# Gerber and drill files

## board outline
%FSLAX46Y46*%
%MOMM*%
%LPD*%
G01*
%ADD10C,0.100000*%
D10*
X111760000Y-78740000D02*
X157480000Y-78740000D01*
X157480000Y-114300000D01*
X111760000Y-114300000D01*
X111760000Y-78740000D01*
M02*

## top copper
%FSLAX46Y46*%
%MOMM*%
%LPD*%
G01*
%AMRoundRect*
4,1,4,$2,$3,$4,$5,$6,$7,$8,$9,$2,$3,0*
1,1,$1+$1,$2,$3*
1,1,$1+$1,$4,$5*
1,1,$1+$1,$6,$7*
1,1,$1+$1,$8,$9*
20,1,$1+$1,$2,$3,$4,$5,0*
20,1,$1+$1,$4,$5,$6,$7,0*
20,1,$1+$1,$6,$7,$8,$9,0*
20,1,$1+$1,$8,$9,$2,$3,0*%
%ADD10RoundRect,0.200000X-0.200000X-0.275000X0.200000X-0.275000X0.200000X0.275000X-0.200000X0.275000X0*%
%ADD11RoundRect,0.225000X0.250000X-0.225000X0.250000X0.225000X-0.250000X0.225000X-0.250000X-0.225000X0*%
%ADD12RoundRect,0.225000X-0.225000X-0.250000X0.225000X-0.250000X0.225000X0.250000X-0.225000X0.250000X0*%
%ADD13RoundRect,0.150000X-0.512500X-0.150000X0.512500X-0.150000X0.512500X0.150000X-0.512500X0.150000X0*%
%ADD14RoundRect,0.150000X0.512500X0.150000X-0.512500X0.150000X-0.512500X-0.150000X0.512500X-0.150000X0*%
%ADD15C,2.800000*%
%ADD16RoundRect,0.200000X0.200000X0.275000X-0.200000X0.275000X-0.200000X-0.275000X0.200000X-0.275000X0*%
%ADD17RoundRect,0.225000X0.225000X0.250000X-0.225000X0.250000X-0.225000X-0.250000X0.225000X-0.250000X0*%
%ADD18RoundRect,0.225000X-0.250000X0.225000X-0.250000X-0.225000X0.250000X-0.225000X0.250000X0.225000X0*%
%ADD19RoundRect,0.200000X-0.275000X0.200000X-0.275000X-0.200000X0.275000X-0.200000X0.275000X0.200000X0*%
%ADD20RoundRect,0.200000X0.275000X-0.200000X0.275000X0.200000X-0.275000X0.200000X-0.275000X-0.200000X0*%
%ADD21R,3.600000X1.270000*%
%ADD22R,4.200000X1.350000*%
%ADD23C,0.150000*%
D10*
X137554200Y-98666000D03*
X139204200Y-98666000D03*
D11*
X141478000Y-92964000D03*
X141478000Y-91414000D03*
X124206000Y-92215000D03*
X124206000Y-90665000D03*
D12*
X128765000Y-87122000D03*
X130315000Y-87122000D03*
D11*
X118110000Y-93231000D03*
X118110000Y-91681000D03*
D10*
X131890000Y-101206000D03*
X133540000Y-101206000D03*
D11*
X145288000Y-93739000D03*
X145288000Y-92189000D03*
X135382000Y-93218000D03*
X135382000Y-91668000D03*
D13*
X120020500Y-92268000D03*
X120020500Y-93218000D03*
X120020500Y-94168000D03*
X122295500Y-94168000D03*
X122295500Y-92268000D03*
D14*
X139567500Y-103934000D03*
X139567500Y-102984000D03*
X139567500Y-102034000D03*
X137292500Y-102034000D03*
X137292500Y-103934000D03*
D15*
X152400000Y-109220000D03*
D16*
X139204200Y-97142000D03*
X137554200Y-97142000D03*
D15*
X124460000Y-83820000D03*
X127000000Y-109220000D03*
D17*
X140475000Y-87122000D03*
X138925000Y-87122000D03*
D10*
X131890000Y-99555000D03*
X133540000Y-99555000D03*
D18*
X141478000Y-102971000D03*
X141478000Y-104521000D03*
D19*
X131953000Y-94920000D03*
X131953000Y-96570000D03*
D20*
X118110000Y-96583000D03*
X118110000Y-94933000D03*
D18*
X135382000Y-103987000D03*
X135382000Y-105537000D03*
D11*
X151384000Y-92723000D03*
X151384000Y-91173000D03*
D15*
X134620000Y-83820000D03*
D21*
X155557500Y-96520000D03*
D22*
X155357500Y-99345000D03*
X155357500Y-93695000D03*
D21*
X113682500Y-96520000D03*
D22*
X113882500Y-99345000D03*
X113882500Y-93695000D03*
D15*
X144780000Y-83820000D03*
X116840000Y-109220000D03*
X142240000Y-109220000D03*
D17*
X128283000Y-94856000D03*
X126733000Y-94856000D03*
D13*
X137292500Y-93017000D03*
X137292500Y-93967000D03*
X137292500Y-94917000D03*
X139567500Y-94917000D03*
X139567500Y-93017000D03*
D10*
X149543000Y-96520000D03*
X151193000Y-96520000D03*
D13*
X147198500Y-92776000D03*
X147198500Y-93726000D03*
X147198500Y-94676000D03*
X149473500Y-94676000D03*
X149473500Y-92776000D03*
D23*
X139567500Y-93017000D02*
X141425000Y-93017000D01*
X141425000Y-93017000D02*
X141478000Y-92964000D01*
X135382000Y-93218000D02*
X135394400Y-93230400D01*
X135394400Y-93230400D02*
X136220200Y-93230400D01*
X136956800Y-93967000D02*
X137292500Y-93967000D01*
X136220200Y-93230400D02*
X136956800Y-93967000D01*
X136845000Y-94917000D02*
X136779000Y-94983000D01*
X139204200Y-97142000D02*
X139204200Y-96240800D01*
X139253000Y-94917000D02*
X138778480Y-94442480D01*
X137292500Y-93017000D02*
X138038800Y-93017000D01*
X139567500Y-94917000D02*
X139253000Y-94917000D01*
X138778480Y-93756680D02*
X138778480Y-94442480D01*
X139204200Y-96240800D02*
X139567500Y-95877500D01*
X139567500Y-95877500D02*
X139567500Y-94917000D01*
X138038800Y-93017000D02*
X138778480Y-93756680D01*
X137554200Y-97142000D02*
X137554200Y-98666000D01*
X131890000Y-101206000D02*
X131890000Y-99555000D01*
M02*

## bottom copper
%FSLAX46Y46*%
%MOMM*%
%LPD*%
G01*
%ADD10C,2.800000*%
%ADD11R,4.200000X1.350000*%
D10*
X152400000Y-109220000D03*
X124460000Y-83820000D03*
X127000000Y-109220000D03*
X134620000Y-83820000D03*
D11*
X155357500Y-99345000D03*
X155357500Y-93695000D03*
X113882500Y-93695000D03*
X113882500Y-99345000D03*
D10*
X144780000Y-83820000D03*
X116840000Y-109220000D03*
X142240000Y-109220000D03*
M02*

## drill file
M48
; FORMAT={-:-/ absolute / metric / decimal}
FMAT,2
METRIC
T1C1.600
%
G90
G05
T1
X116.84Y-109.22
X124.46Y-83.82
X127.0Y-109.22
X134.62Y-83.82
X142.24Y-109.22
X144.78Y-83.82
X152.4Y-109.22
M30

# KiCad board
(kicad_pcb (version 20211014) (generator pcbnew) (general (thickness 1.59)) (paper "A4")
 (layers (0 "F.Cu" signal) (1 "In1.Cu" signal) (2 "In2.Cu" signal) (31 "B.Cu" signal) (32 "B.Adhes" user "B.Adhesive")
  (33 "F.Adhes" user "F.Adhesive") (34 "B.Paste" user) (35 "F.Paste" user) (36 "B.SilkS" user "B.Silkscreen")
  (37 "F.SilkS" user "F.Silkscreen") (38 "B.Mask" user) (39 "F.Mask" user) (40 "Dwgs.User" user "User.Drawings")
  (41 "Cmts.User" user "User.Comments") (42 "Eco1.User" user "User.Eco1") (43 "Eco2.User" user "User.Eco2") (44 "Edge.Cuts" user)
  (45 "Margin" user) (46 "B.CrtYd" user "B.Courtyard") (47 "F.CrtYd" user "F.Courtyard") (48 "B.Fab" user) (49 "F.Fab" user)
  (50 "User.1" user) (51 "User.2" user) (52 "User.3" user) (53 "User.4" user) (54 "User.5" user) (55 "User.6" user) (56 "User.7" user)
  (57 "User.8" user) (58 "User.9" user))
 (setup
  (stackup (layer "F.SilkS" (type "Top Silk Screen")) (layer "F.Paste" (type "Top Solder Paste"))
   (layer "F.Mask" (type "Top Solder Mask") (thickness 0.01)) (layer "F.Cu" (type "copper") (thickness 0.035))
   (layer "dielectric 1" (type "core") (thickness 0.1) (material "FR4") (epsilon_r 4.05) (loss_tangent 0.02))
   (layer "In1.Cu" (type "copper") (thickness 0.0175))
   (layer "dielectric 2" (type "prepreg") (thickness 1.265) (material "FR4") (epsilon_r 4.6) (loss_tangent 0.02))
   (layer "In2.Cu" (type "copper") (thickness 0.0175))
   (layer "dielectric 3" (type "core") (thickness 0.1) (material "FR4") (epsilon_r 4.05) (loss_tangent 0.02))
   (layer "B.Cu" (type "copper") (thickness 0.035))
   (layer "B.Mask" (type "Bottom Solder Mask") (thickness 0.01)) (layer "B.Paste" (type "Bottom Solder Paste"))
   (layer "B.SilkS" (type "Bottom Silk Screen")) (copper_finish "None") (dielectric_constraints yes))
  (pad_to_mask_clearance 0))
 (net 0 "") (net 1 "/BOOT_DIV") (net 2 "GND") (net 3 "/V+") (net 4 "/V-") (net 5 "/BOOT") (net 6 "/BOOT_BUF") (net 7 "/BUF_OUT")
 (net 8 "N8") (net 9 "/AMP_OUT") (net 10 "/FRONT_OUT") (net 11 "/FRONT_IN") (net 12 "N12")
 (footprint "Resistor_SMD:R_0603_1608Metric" (layer "F.Cu") (at 138.3792 98.666)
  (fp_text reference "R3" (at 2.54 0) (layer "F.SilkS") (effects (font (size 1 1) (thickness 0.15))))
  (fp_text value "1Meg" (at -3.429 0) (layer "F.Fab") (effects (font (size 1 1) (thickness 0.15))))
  (pad "1" smd roundrect (at -0.825 0) (size 0.8 0.95) (layers "F.Cu" "F.Paste" "F.Mask") (roundrect_rratio 0.25) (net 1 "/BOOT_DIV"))
  (pad "2" smd roundrect (at 0.825 0) (size 0.8 0.95) (layers "F.Cu" "F.Paste" "F.Mask") (roundrect_rratio 0.25) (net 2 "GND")))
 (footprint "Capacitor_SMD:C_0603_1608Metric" (layer "F.Cu") (at 141.478 92.189 90)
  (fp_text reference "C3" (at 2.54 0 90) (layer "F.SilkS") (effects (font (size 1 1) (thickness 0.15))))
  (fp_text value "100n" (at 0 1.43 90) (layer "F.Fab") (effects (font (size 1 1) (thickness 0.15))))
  (pad "1" smd roundrect (at -0.775 0 90) (size 0.9 0.95) (layers "F.Cu" "F.Paste" "F.Mask") (roundrect_rratio 0.25) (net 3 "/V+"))
  (pad "2" smd roundrect (at 0.775 0 90) (size 0.9 0.95) (layers "F.Cu" "F.Paste" "F.Mask") (roundrect_rratio 0.25) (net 2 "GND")))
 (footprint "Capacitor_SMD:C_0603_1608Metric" (layer "F.Cu") (at 124.206 91.44 90)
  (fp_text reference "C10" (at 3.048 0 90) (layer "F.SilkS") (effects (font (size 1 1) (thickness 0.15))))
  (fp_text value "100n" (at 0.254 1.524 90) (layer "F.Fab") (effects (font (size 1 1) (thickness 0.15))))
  (pad "1" smd roundrect (at -0.775 0 90) (size 0.9 0.95) (layers "F.Cu" "F.Paste" "F.Mask") (roundrect_rratio 0.25) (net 3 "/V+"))
  (pad "2" smd roundrect (at 0.775 0 90) (size 0.9 0.95) (layers "F.Cu" "F.Paste" "F.Mask") (roundrect_rratio 0.25) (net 2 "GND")))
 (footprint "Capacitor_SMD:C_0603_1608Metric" (layer "F.Cu") (at 129.54 87.122)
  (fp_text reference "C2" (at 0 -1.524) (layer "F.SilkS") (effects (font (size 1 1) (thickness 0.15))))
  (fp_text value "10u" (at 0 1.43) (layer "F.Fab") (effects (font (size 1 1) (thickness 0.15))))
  (pad "1" smd roundrect (at -0.775 0) (size 0.9 0.95) (layers "F.Cu" "F.Paste" "F.Mask") (roundrect_rratio 0.25) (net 3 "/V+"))
  (pad "2" smd roundrect (at 0.775 0) (size 0.9 0.95) (layers "F.Cu" "F.Paste" "F.Mask") (roundrect_rratio 0.25) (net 2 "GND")))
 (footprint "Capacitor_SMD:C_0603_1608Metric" (layer "F.Cu") (at 118.11 92.456 90)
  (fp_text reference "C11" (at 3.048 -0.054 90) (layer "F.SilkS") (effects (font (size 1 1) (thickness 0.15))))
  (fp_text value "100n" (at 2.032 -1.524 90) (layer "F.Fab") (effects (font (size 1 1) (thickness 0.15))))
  (pad "1" smd roundrect (at -0.775 0 90) (size 0.9 0.95) (layers "F.Cu" "F.Paste" "F.Mask") (roundrect_rratio 0.25) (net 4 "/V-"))
  (pad "2" smd roundrect (at 0.775 0 90) (size 0.9 0.95) (layers "F.Cu" "F.Paste" "F.Mask") (roundrect_rratio 0.25) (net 2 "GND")))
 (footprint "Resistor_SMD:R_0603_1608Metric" (layer "F.Cu") (at 132.715 101.206)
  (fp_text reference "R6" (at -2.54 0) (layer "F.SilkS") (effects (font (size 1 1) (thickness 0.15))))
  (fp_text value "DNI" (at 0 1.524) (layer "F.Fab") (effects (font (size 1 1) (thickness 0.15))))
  (pad "1" smd roundrect (at -0.825 0) (size 0.8 0.95) (layers "F.Cu" "F.Paste" "F.Mask") (roundrect_rratio 0.25) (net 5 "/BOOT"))
  (pad "2" smd roundrect (at 0.825 0) (size 0.8 0.95) (layers "F.Cu" "F.Paste" "F.Mask") (roundrect_rratio 0.25) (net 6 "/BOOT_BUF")))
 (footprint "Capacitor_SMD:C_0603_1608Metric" (layer "F.Cu") (at 145.288 92.964 90)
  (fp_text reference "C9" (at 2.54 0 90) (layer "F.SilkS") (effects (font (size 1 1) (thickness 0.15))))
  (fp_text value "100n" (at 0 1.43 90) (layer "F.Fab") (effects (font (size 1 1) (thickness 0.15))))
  (pad "1" smd roundrect (at -0.775 0 90) (size 0.9 0.95) (layers "F.Cu" "F.Paste" "F.Mask") (roundrect_rratio 0.25) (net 4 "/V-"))
  (pad "2" smd roundrect (at 0.775 0 90) (size 0.9 0.95) (layers "F.Cu" "F.Paste" "F.Mask") (roundrect_rratio 0.25) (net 2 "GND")))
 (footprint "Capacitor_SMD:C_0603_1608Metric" (layer "F.Cu") (at 135.382 92.443 90)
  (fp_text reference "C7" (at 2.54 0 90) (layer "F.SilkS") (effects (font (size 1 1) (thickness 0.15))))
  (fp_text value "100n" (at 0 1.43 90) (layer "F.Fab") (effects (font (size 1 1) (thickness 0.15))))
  (pad "1" smd roundrect (at -0.775 0 90) (size 0.9 0.95) (layers "F.Cu" "F.Paste" "F.Mask") (roundrect_rratio 0.25) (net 4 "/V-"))
  (pad "2" smd roundrect (at 0.775 0 90) (size 0.9 0.95) (layers "F.Cu" "F.Paste" "F.Mask") (roundrect_rratio 0.25) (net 2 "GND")))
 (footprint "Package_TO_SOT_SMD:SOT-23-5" (layer "F.Cu") (at 121.158 93.218)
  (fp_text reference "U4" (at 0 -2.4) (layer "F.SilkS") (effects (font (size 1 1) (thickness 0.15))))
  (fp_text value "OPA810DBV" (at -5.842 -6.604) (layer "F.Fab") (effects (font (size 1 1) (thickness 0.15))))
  (pad "1" smd roundrect (at -1.1375 -0.95) (size 1.325 0.6) (layers "F.Cu" "F.Paste" "F.Mask") (roundrect_rratio 0.25) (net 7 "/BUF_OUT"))
  (pad "2" smd roundrect (at -1.1375 0) (size 1.325 0.6) (layers "F.Cu" "F.Paste" "F.Mask") (roundrect_rratio 0.25) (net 4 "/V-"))
  (pad "3" smd roundrect (at -1.1375 0.95) (size 1.325 0.6) (layers "F.Cu" "F.Paste" "F.Mask") (roundrect_rratio 0.25) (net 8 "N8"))
  (pad "4" smd roundrect (at 1.1375 0.95) (size 1.325 0.6) (layers "F.Cu" "F.Paste" "F.Mask") (roundrect_rratio 0.25) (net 7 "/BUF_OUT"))
  (pad "5" smd roundrect (at 1.1375 -0.95) (size 1.325 0.6) (layers "F.Cu" "F.Paste" "F.Mask") (roundrect_rratio 0.25) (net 3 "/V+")))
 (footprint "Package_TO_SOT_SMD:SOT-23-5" (layer "F.Cu") (at 138.43 102.984 180)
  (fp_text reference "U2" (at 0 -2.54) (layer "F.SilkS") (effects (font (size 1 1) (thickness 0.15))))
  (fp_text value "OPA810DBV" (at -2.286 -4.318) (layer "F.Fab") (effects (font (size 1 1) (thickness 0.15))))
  (pad "1" smd roundrect (at -1.1375 -0.95 180) (size 1.325 0.6) (layers "F.Cu" "F.Paste" "F.Mask") (roundrect_rratio 0.25)
   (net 6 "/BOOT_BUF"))
  (pad "2" smd roundrect (at -1.1375 0 180) (size 1.325 0.6) (layers "F.Cu" "F.Paste" "F.Mask") (roundrect_rratio 0.25) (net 4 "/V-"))
  (pad "3" smd roundrect (at -1.1375 0.95 180) (size 1.325 0.6) (layers "F.Cu" "F.Paste" "F.Mask") (roundrect_rratio 0.25)
   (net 1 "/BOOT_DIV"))
  (pad "4" smd roundrect (at 1.1375 0.95 180) (size 1.325 0.6) (layers "F.Cu" "F.Paste" "F.Mask") (roundrect_rratio 0.25)
   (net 6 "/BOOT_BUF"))
  (pad "5" smd roundrect (at 1.1375 -0.95 180) (size 1.325 0.6) (layers "F.Cu" "F.Paste" "F.Mask") (roundrect_rratio 0.25) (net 3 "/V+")))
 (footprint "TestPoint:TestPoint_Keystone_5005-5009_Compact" (layer "F.Cu") (at 152.4 109.22)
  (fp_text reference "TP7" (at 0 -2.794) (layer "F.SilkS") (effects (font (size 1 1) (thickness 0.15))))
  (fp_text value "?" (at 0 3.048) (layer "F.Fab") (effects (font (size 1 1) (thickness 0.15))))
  (pad "1" thru_hole circle (at 0 0) (size 2.8 2.8) (drill 1.6) (layers *.Cu *.Mask) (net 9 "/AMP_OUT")))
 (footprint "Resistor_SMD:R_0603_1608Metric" (layer "F.Cu") (at 138.3792 97.142 180)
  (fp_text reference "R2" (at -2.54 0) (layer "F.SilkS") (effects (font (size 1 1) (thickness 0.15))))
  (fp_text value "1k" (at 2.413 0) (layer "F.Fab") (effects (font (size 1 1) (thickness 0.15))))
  (pad "1" smd roundrect (at -0.825 0 180) (size 0.8 0.95) (layers "F.Cu" "F.Paste" "F.Mask") (roundrect_rratio 0.25) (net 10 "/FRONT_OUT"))
  (pad "2" smd roundrect (at 0.825 0 180) (size 0.8 0.95) (layers "F.Cu" "F.Paste" "F.Mask") (roundrect_rratio 0.25) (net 1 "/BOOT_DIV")))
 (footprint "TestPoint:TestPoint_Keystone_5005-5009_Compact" (layer "F.Cu") (at 124.46 83.82)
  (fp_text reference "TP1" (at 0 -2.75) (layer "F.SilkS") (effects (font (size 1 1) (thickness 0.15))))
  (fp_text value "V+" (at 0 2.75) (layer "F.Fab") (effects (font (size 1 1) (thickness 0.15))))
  (pad "1" thru_hole circle (at 0 0) (size 2.8 2.8) (drill 1.6) (layers *.Cu *.Mask) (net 3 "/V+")))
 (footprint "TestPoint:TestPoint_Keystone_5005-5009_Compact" (layer "F.Cu") (at 127 109.22)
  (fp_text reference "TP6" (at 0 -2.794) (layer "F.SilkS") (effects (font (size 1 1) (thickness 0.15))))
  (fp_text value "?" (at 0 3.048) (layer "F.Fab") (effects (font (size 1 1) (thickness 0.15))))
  (pad "1" thru_hole circle (at 0 0) (size 2.8 2.8) (drill 1.6) (layers *.Cu *.Mask) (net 6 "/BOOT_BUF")))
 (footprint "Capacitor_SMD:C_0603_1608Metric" (layer "F.Cu") (at 139.7 87.122 180)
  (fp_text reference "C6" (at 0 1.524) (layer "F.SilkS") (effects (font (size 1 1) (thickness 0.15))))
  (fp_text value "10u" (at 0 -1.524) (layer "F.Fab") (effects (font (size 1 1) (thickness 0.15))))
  (pad "1" smd roundrect (at -0.775 0 180) (size 0.9 0.95) (layers "F.Cu" "F.Paste" "F.Mask") (roundrect_rratio 0.25) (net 4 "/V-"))
  (pad "2" smd roundrect (at 0.775 0 180) (size 0.9 0.95) (layers "F.Cu" "F.Paste" "F.Mask") (roundrect_rratio 0.25) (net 2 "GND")))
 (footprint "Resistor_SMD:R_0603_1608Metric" (layer "F.Cu") (at 132.715 99.555)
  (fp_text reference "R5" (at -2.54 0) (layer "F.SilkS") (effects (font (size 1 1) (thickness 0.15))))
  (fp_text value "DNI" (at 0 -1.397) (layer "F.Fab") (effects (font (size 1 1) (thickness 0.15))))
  (pad "1" smd roundrect (at -0.825 0) (size 0.8 0.95) (layers "F.Cu" "F.Paste" "F.Mask") (roundrect_rratio 0.25) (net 5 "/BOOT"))
  (pad "2" smd roundrect (at 0.825 0) (size 0.8 0.95) (layers "F.Cu" "F.Paste" "F.Mask") (roundrect_rratio 0.25) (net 1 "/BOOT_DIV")))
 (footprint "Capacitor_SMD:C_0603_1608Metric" (layer "F.Cu") (at 141.478 103.746 -90)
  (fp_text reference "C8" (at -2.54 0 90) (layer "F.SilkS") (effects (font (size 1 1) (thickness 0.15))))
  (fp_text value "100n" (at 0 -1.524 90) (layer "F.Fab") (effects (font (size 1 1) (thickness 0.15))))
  (pad "1" smd roundrect (at -0.775 0 270) (size 0.9 0.95) (layers "F.Cu" "F.Paste" "F.Mask") (roundrect_rratio 0.25) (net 4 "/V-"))
  (pad "2" smd roundrect (at 0.775 0 270) (size 0.9 0.95) (layers "F.Cu" "F.Paste" "F.Mask") (roundrect_rratio 0.25) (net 2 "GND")))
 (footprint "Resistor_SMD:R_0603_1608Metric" (layer "F.Cu") (at 131.953 95.745 -90)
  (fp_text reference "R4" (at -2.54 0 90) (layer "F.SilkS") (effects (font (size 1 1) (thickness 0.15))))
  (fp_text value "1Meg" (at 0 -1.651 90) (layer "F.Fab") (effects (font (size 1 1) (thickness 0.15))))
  (pad "1" smd roundrect (at -0.825 0 270) (size 0.8 0.95) (layers "F.Cu" "F.Paste" "F.Mask") (roundrect_rratio 0.25) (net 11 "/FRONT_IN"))
  (pad "2" smd roundrect (at 0.825 0 270) (size 0.8 0.95) (layers "F.Cu" "F.Paste" "F.Mask") (roundrect_rratio 0.25) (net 5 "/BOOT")))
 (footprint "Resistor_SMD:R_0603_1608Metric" (layer "F.Cu") (at 118.11 95.758 90)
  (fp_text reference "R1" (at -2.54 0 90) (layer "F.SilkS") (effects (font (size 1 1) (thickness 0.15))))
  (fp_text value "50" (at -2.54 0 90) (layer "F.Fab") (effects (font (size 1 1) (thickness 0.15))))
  (pad "1" smd roundrect (at -0.825 0 90) (size 0.8 0.95) (layers "F.Cu" "F.Paste" "F.Mask") (roundrect_rratio 0.25) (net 8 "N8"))
  (pad "2" smd roundrect (at 0.825 0 90) (size 0.8 0.95) (layers "F.Cu" "F.Paste" "F.Mask") (roundrect_rratio 0.25) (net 2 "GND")))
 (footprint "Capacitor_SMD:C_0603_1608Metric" (layer "F.Cu") (at 135.382 104.762 -90)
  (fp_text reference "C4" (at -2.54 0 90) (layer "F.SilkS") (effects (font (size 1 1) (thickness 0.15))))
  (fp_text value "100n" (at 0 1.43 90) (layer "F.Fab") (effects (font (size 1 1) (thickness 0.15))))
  (pad "1" smd roundrect (at -0.775 0 270) (size 0.9 0.95) (layers "F.Cu" "F.Paste" "F.Mask") (roundrect_rratio 0.25) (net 3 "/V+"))
  (pad "2" smd roundrect (at 0.775 0 270) (size 0.9 0.95) (layers "F.Cu" "F.Paste" "F.Mask") (roundrect_rratio 0.25) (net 2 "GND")))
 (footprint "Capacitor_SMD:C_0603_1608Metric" (layer "F.Cu") (at 151.384 91.948 90)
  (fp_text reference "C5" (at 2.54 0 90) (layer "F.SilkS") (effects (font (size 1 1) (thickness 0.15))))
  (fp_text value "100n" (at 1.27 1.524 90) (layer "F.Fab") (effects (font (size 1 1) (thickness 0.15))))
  (pad "1" smd roundrect (at -0.775 0 90) (size 0.9 0.95) (layers "F.Cu" "F.Paste" "F.Mask") (roundrect_rratio 0.25) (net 3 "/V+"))
  (pad "2" smd roundrect (at 0.775 0 90) (size 0.9 0.95) (layers "F.Cu" "F.Paste" "F.Mask") (roundrect_rratio 0.25) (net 2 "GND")))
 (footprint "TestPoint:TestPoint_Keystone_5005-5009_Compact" (layer "F.Cu") (at 134.62 83.82)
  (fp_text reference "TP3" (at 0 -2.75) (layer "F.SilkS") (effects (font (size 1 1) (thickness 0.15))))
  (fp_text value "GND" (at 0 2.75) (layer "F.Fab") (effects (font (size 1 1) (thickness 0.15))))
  (pad "1" thru_hole circle (at 0 0) (size 2.8 2.8) (drill 1.6) (layers *.Cu *.Mask) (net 2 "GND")))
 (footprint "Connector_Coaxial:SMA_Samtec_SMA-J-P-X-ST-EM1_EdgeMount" (layer "F.Cu") (at 155.3575 96.52 90)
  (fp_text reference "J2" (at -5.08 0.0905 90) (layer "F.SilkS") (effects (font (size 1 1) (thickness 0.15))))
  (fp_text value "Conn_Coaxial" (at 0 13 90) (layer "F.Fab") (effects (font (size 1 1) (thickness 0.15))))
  (pad "1" smd rect (at 0 0.2 90) (size 1.27 3.6) (layers "F.Cu" "F.Paste" "F.Mask") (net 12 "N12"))
  (pad "2" smd rect (at -2.825 0 90) (size 1.35 4.2) (layers "F.Cu" "F.Paste" "F.Mask") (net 2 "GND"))
  (pad "2" smd rect (at 2.825 0 90) (size 1.35 4.2) (layers "F.Cu" "F.Paste" "F.Mask") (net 2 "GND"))
  (pad "2" smd rect (at -2.825 0 90) (size 1.35 4.2) (layers "B.Cu" "B.Paste" "B.Mask") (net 2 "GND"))
  (pad "2" smd rect (at 2.825 0 90) (size 1.35 4.2) (layers "B.Cu" "B.Paste" "B.Mask") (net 2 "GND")))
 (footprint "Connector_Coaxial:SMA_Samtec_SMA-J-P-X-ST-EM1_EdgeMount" (layer "F.Cu") (at 113.8825 96.52 -90)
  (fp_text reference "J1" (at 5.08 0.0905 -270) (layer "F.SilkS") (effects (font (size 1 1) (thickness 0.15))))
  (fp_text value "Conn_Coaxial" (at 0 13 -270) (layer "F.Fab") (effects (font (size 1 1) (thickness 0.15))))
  (pad "1" smd rect (at 0 0.2 270) (size 1.27 3.6) (layers "F.Cu" "F.Paste" "F.Mask") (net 8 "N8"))
  (pad "2" smd rect (at 2.825 0 270) (size 1.35 4.2) (layers "F.Cu" "F.Paste" "F.Mask") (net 2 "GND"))
  (pad "2" smd rect (at -2.825 0 270) (size 1.35 4.2) (layers "B.Cu" "B.Paste" "B.Mask") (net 2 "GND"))
  (pad "2" smd rect (at -2.825 0 270) (size 1.35 4.2) (layers "F.Cu" "F.Paste" "F.Mask") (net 2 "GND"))
  (pad "2" smd rect (at 2.825 0 270) (size 1.35 4.2) (layers "B.Cu" "B.Paste" "B.Mask") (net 2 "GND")))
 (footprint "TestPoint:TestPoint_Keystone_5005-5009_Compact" (layer "F.Cu") (at 144.78 83.82)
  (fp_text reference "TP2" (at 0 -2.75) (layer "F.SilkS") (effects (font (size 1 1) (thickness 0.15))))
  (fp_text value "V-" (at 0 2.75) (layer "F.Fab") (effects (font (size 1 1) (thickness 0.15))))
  (pad "1" thru_hole circle (at 0 0) (size 2.8 2.8) (drill 1.6) (layers *.Cu *.Mask) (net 4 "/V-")))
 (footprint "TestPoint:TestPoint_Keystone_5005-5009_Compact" (layer "F.Cu") (at 116.84 109.22)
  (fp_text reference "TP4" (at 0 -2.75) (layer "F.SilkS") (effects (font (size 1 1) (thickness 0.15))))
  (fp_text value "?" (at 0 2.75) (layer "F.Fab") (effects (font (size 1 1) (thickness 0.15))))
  (pad "1" thru_hole circle (at 0 0) (size 2.8 2.8) (drill 1.6) (layers *.Cu *.Mask) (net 7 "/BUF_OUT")))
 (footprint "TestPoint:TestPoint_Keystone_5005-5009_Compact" (layer "F.Cu") (at 142.24 109.22)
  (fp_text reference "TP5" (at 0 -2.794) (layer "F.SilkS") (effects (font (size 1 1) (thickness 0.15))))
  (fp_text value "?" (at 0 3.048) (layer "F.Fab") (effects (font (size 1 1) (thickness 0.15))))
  (pad "1" thru_hole circle (at 0 0) (size 2.8 2.8) (drill 1.6) (layers *.Cu *.Mask) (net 10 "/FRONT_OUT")))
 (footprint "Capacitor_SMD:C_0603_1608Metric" (layer "F.Cu") (at 127.508 94.856 180)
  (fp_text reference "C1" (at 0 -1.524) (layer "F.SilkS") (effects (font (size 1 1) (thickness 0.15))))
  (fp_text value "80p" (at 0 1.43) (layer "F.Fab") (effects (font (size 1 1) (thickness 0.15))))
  (pad "1" smd roundrect (at -0.775 0 180) (size 0.9 0.95) (layers "F.Cu" "F.Paste" "F.Mask") (roundrect_rratio 0.25) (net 11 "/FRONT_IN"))
  (pad "2" smd roundrect (at 0.775 0 180) (size 0.9 0.95) (layers "F.Cu" "F.Paste" "F.Mask") (roundrect_rratio 0.25) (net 7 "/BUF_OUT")))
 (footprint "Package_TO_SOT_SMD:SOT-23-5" (layer "F.Cu") (at 138.43 93.967)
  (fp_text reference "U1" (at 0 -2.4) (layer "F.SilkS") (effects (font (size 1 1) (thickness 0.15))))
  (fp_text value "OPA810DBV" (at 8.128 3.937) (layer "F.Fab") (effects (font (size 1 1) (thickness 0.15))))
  (pad "1" smd roundrect (at -1.1375 -0.95) (size 1.325 0.6) (layers "F.Cu" "F.Paste" "F.Mask") (roundrect_rratio 0.25)
   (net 10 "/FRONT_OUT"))
  (pad "2" smd roundrect (at -1.1375 0) (size 1.325 0.6) (layers "F.Cu" "F.Paste" "F.Mask") (roundrect_rratio 0.25) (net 4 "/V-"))
  (pad "3" smd roundrect (at -1.1375 0.95) (size 1.325 0.6) (layers "F.Cu" "F.Paste" "F.Mask") (roundrect_rratio 0.25) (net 11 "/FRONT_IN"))
  (pad "4" smd roundrect (at 1.1375 0.95) (size 1.325 0.6) (layers "F.Cu" "F.Paste" "F.Mask") (roundrect_rratio 0.25) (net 10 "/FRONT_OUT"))
  (pad "5" smd roundrect (at 1.1375 -0.95) (size 1.325 0.6) (layers "F.Cu" "F.Paste" "F.Mask") (roundrect_rratio 0.25) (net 3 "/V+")))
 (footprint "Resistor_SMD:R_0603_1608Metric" (layer "F.Cu") (at 150.368 96.52)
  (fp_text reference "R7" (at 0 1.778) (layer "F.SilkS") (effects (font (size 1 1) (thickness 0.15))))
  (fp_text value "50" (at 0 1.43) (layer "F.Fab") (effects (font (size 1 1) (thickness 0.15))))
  (pad "1" smd roundrect (at -0.825 0) (size 0.8 0.95) (layers "F.Cu" "F.Paste" "F.Mask") (roundrect_rratio 0.25) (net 9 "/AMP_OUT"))
  (pad "2" smd roundrect (at 0.825 0) (size 0.8 0.95) (layers "F.Cu" "F.Paste" "F.Mask") (roundrect_rratio 0.25) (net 12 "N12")))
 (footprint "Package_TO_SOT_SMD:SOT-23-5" (layer "F.Cu") (at 148.336 93.726)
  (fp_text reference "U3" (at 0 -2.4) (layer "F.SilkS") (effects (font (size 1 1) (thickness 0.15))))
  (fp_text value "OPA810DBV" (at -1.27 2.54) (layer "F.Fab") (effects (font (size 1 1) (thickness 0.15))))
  (pad "1" smd roundrect (at -1.1375 -0.95) (size 1.325 0.6) (layers "F.Cu" "F.Paste" "F.Mask") (roundrect_rratio 0.25) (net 9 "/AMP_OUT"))
  (pad "2" smd roundrect (at -1.1375 0) (size 1.325 0.6) (layers "F.Cu" "F.Paste" "F.Mask") (roundrect_rratio 0.25) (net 4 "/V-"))
  (pad "3" smd roundrect (at -1.1375 0.95) (size 1.325 0.6) (layers "F.Cu" "F.Paste" "F.Mask") (roundrect_rratio 0.25) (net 10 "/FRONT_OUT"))
  (pad "4" smd roundrect (at 1.1375 0.95) (size 1.325 0.6) (layers "F.Cu" "F.Paste" "F.Mask") (roundrect_rratio 0.25) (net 9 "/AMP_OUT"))
  (pad "5" smd roundrect (at 1.1375 -0.95) (size 1.325 0.6) (layers "F.Cu" "F.Paste" "F.Mask") (roundrect_rratio 0.25) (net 3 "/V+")))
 (gr_rect (start 111.76 78.74) (end 157.48 114.3) (layer "Edge.Cuts") (width 0.1) (fill none))
 (segment (start 139.5675 93.017) (end 141.425 93.017) (width 0.15) (layer "F.Cu") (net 3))
 (segment (start 141.425 93.017) (end 141.478 92.964) (width 0.15) (layer "F.Cu") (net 3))
 (segment (start 135.382 93.218) (end 135.3944 93.2304) (width 0.15) (layer "F.Cu") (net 4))
 (segment (start 135.3944 93.2304) (end 136.2202 93.2304) (width 0.15) (layer "F.Cu") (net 4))
 (segment (start 136.9568 93.967) (end 137.2925 93.967) (width 0.15) (layer "F.Cu") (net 4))
 (segment (start 136.2202 93.2304) (end 136.9568 93.967) (width 0.15) (layer "F.Cu") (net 4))
 (segment (start 136.845 94.917) (end 136.779 94.983) (width 0.15) (layer "F.Cu") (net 11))
 (segment (start 139.2042 97.142) (end 139.2042 96.2408) (width 0.15) (layer "F.Cu") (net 10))
 (segment (start 139.253 94.917) (end 138.77848 94.44248) (width 0.15) (layer "F.Cu") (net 10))
 (segment (start 137.2925 93.017) (end 138.0388 93.017) (width 0.15) (layer "F.Cu") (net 10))
 (segment (start 139.5675 94.917) (end 139.253 94.917) (width 0.15) (layer "F.Cu") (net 10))
 (segment (start 138.77848 93.75668) (end 138.77848 94.44248) (width 0.15) (layer "F.Cu") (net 10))
 (segment (start 139.2042 96.2408) (end 139.5675 95.8775) (width 0.15) (layer "F.Cu") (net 10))
 (segment (start 139.5675 95.8775) (end 139.5675 94.917) (width 0.15) (layer "F.Cu") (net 10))
 (segment (start 138.0388 93.017) (end 138.77848 93.75668) (width 0.15) (layer "F.Cu") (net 10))
 (segment (start 137.5542 97.142) (end 137.5542 98.666) (width 0.15) (layer "F.Cu") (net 1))
 (segment (start 131.89 101.206) (end 131.89 99.555) (width 0.15) (layer "F.Cu") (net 5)))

